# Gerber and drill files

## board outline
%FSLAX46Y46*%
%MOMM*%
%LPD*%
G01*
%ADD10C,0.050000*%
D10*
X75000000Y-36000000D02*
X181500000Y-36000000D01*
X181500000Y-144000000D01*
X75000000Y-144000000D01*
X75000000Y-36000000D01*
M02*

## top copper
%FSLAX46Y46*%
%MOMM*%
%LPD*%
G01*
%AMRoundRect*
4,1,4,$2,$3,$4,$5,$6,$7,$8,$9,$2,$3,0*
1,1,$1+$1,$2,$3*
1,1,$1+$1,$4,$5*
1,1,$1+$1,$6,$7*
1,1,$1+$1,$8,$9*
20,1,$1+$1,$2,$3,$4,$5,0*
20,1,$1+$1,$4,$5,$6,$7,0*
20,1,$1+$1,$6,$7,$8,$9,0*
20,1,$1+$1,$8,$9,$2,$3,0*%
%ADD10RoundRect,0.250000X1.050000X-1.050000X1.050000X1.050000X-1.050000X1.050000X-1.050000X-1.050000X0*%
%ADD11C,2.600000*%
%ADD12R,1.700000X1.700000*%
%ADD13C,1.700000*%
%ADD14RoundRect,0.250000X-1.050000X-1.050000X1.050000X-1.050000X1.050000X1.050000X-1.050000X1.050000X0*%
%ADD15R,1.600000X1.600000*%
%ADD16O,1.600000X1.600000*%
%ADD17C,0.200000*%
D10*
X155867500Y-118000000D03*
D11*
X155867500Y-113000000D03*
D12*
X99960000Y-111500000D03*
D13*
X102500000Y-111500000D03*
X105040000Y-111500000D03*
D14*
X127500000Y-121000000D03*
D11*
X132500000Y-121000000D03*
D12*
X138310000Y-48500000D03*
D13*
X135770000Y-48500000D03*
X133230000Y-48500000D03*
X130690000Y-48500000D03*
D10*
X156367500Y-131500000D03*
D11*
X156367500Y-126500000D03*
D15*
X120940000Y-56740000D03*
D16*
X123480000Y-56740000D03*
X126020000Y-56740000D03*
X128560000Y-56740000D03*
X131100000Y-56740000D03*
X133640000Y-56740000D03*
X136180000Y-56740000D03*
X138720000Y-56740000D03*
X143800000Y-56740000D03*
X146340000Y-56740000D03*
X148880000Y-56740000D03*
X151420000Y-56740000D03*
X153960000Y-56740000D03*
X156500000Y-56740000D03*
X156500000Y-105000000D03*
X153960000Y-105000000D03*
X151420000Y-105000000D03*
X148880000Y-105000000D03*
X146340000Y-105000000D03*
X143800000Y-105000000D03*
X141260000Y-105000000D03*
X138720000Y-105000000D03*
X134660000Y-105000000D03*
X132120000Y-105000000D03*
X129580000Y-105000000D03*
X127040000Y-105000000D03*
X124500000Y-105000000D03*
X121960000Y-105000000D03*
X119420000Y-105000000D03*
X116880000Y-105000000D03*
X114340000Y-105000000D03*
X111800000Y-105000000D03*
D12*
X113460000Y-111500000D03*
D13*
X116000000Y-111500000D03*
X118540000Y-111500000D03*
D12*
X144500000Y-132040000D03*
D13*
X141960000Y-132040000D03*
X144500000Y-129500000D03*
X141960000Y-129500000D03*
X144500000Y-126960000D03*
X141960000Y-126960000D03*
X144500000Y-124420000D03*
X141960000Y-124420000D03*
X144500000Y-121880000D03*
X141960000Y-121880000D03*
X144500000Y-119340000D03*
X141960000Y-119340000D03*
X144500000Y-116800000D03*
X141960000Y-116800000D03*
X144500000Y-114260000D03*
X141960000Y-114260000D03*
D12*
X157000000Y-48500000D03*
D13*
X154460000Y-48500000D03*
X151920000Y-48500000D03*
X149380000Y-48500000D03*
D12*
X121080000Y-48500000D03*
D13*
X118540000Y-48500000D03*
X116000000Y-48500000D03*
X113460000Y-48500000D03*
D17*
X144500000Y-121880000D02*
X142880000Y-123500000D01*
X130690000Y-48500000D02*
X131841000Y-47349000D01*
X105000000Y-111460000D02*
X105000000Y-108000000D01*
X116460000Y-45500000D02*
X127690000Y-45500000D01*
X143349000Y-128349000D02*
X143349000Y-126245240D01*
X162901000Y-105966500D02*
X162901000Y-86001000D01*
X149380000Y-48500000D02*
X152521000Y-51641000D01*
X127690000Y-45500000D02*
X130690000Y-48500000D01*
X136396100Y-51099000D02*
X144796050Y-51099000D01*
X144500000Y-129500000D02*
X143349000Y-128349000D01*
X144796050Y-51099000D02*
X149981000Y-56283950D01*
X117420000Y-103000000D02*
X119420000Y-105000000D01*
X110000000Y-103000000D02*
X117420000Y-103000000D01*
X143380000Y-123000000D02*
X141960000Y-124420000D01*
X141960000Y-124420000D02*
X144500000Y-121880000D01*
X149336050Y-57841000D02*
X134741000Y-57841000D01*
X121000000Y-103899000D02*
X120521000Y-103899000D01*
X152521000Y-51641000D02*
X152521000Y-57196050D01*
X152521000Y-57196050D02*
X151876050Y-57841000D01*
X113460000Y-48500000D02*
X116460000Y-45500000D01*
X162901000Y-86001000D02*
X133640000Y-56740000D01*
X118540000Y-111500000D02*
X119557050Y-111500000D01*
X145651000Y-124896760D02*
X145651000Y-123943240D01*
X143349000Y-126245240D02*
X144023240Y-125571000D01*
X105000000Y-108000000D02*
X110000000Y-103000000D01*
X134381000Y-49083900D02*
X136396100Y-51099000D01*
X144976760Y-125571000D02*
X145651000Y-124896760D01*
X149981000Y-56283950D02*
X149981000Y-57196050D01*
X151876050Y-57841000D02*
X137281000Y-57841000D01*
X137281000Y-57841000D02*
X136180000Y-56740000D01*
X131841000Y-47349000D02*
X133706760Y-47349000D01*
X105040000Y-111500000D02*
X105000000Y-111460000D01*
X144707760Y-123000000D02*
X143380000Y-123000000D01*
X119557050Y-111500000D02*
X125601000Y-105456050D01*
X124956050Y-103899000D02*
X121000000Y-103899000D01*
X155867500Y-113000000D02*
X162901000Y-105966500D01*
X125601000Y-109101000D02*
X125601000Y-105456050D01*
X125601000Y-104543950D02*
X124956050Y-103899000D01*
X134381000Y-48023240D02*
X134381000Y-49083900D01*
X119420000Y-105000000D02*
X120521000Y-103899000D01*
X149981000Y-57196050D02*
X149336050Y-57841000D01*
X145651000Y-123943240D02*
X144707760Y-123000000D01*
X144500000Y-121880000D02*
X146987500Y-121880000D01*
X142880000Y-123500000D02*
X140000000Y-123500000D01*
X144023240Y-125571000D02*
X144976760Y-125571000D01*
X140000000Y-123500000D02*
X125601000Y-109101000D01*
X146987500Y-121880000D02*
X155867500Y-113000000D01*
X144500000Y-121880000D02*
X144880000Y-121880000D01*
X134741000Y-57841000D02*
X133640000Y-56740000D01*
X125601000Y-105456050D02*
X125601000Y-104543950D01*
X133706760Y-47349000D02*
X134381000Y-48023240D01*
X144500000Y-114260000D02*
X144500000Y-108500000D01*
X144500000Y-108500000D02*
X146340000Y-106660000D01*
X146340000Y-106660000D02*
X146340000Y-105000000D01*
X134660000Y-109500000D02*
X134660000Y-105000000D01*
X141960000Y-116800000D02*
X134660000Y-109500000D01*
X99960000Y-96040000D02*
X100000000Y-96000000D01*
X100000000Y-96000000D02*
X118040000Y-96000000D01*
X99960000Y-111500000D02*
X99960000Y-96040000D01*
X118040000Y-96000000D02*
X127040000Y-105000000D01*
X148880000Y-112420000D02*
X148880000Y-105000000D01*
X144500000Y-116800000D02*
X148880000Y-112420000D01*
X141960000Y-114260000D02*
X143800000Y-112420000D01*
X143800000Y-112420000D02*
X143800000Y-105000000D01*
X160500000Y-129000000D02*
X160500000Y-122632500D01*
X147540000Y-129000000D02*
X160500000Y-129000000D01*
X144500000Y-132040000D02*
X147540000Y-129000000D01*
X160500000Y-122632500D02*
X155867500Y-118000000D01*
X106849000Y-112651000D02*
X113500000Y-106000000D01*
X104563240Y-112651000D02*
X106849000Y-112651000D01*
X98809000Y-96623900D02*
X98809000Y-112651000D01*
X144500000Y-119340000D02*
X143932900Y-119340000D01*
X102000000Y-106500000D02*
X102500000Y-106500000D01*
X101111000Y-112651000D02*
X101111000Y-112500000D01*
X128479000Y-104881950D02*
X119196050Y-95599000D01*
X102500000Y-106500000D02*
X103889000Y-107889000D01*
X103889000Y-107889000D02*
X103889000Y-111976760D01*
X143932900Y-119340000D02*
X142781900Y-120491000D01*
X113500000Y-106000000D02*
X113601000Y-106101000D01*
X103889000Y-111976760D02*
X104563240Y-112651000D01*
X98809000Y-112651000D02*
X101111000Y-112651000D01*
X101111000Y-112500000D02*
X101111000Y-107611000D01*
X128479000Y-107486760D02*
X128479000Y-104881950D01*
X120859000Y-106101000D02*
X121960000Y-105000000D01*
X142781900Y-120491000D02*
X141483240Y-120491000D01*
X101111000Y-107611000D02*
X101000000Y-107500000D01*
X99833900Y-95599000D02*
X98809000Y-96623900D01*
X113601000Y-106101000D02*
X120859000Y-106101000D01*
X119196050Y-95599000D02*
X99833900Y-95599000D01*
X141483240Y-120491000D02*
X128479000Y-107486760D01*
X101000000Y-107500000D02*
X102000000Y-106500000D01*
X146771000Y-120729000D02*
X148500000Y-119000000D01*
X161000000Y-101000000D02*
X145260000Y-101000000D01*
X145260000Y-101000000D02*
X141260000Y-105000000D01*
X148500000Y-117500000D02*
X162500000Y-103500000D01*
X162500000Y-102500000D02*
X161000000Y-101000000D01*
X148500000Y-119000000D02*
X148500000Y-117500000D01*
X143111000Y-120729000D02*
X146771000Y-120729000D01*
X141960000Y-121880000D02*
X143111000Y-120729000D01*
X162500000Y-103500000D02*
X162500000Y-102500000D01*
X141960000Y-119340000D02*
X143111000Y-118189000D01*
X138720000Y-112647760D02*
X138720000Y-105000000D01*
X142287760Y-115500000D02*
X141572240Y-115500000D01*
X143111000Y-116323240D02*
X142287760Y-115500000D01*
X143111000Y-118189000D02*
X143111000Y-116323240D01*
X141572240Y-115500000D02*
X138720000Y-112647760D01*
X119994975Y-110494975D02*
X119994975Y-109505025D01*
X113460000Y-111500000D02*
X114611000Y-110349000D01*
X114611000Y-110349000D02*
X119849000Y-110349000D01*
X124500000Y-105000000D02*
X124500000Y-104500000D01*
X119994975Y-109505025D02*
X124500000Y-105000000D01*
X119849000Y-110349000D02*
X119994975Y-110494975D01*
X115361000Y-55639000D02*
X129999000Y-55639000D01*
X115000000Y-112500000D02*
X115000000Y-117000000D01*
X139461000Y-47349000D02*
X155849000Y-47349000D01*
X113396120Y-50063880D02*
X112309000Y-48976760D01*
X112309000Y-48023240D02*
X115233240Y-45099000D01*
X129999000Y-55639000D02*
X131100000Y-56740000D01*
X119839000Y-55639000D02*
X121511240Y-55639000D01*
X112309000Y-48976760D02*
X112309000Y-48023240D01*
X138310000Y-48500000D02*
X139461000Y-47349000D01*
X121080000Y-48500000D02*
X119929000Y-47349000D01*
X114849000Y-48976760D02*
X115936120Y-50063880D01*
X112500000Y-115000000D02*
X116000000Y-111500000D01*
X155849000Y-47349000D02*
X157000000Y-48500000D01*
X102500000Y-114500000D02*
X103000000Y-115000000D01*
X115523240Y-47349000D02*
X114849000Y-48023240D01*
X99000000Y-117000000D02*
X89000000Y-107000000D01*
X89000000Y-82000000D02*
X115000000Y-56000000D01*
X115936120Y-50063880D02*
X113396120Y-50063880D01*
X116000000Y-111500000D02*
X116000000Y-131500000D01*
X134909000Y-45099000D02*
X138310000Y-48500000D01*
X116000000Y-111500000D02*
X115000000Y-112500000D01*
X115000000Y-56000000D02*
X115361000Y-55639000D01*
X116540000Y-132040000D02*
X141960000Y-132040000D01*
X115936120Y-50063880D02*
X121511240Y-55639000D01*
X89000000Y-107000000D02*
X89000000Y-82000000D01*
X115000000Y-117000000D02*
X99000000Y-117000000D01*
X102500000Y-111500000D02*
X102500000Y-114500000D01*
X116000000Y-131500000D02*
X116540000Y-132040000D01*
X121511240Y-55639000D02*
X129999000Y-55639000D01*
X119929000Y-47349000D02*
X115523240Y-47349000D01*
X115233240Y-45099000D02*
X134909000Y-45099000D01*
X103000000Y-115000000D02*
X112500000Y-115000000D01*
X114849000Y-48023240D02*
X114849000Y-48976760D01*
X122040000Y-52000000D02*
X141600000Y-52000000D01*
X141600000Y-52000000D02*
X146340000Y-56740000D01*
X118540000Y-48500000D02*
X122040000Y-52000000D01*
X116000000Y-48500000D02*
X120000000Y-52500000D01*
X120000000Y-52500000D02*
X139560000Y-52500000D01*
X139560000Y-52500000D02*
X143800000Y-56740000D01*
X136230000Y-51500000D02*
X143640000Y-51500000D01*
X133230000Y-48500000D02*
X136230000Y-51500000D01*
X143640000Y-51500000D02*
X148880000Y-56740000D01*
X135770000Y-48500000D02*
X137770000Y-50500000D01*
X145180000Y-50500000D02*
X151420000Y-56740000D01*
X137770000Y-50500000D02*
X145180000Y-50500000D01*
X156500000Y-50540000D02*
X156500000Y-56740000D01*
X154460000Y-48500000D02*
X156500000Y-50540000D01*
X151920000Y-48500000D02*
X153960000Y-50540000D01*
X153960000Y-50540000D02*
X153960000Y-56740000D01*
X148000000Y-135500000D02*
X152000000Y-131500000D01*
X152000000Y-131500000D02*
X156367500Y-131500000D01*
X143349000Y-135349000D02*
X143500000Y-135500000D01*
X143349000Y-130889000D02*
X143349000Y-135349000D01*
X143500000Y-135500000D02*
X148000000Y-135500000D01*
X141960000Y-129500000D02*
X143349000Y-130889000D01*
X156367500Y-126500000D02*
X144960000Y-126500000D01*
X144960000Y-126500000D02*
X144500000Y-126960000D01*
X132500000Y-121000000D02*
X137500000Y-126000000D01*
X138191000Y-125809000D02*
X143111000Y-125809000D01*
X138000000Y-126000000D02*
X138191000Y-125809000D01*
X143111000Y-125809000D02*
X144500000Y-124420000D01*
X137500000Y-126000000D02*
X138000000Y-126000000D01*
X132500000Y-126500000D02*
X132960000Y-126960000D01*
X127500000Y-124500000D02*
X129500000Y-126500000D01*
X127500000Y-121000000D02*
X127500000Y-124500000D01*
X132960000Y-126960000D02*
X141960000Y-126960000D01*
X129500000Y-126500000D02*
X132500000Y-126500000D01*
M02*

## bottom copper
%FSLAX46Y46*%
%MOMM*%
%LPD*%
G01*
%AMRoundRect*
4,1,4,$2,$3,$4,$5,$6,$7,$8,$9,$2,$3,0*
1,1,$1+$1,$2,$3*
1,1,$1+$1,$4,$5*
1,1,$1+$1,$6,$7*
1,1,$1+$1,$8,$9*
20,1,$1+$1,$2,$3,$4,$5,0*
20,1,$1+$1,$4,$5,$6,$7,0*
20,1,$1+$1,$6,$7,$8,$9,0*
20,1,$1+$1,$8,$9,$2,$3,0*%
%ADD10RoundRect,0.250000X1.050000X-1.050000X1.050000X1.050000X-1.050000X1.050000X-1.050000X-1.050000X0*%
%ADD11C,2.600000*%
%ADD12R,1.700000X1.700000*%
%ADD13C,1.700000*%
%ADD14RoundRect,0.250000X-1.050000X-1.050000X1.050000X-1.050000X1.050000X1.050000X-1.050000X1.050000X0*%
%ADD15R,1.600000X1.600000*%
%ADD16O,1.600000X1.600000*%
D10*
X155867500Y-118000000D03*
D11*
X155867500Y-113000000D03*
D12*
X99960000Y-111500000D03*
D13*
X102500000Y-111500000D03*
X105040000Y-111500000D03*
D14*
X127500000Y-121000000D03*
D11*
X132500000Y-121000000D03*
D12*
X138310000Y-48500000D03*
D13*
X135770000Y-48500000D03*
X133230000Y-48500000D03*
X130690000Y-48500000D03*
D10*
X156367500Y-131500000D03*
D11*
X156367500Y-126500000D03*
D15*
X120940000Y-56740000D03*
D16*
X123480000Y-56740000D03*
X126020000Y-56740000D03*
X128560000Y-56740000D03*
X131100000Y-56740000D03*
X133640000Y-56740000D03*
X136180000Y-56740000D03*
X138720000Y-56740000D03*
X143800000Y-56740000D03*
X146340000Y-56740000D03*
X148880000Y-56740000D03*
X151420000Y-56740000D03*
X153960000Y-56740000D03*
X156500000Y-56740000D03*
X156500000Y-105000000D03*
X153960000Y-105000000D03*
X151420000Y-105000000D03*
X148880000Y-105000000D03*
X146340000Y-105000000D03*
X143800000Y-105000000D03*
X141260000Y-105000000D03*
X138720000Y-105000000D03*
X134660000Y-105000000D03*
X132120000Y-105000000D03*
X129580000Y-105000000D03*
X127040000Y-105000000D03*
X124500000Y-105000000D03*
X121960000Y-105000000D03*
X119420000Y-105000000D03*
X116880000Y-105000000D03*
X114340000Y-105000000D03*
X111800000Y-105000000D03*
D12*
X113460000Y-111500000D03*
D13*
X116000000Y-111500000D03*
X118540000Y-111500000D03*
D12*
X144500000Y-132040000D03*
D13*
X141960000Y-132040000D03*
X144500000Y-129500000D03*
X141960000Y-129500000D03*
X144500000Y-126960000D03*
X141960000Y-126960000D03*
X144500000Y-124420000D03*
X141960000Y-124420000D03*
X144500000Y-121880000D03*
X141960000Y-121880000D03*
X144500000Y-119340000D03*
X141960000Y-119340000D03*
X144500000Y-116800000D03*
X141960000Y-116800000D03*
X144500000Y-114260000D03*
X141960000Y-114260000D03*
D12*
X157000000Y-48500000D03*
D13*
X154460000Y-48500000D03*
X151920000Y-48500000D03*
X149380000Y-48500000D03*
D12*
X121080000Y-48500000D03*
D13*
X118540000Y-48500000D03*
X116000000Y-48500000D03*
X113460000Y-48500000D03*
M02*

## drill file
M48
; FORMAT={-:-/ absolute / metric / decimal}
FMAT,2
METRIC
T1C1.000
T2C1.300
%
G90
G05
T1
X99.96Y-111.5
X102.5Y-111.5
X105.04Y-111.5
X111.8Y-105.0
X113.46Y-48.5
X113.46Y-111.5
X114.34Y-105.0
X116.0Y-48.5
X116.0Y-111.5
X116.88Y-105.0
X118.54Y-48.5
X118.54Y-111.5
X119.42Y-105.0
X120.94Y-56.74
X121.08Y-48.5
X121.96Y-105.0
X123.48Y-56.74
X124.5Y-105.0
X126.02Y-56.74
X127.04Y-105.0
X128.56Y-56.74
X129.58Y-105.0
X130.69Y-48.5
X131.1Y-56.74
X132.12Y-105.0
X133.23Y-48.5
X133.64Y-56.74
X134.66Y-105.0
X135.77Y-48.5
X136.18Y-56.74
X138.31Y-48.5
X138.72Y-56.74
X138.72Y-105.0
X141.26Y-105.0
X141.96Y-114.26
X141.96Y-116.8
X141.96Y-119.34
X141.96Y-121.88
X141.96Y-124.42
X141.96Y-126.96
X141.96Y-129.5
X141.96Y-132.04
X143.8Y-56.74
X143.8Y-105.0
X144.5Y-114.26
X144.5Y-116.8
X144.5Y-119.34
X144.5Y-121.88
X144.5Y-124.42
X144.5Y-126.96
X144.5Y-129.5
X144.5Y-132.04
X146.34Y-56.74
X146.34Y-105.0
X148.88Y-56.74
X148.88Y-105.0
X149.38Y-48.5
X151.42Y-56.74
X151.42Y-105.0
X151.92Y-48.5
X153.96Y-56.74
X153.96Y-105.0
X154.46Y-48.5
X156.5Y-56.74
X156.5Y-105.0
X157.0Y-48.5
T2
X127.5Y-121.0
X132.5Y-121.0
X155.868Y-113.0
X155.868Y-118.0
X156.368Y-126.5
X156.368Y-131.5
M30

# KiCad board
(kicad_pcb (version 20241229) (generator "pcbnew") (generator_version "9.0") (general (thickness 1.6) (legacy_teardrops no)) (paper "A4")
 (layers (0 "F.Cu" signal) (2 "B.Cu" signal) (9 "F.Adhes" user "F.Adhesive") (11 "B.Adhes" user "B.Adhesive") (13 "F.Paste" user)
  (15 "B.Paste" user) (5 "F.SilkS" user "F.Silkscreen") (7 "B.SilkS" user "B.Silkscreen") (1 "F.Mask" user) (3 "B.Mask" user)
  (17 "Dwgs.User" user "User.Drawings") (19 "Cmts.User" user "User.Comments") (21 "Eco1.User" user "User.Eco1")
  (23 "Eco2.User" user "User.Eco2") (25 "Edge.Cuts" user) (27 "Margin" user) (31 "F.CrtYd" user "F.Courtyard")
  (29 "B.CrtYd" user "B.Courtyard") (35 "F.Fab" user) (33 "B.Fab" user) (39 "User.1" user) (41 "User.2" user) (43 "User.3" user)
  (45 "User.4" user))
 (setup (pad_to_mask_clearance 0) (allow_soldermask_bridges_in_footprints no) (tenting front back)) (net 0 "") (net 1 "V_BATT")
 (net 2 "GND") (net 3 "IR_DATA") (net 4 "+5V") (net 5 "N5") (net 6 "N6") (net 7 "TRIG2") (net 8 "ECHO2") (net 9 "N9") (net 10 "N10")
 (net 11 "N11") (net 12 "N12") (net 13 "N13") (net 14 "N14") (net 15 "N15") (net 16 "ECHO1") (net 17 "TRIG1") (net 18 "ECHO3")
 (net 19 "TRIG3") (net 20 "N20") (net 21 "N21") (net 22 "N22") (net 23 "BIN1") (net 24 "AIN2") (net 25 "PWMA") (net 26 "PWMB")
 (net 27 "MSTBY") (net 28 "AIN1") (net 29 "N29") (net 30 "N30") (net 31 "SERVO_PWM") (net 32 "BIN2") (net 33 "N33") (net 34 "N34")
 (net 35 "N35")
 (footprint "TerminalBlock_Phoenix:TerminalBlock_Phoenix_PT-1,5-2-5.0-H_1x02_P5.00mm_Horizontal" (layer "F.Cu") (at 155.8675 118 90)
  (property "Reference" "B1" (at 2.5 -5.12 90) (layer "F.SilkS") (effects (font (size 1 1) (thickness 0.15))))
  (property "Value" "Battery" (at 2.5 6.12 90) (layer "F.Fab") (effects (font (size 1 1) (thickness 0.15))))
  (pad "1" thru_hole roundrect (at 0 0 90) (size 2.6 2.6) (drill 1.3) (layers "*.Cu" "*.Mask") (remove_unused_layers no)
   (roundrect_rratio 0.096154) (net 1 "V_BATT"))
  (pad "2" thru_hole circle (at 5 0 90) (size 2.6 2.6) (drill 1.3) (layers "*.Cu" "*.Mask") (remove_unused_layers no) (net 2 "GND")))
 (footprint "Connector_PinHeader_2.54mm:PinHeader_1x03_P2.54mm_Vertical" (layer "F.Cu") (at 99.96 111.5 90)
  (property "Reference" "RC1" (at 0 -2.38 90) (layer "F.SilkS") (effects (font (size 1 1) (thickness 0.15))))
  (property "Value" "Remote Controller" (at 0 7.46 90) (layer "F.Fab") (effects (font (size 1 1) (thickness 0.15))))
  (pad "1" thru_hole rect (at 0 0 90) (size 1.7 1.7) (drill 1) (layers "*.Cu" "*.Mask") (remove_unused_layers no) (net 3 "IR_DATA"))
  (pad "2" thru_hole circle (at 0 2.54 90) (size 1.7 1.7) (drill 1) (layers "*.Cu" "*.Mask") (remove_unused_layers no) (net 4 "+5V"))
  (pad "3" thru_hole circle (at 0 5.08 90) (size 1.7 1.7) (drill 1) (layers "*.Cu" "*.Mask") (remove_unused_layers no) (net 2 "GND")))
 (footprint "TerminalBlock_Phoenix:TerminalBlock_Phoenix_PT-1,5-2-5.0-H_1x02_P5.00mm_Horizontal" (layer "F.Cu") (at 127.5 121)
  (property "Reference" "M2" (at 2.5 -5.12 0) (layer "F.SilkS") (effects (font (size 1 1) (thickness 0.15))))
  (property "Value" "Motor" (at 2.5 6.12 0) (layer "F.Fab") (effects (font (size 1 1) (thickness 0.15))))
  (pad "1" thru_hole roundrect (at 0 0) (size 2.6 2.6) (drill 1.3) (layers "*.Cu" "*.Mask") (remove_unused_layers no)
   (roundrect_rratio 0.096154) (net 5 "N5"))
  (pad "2" thru_hole circle (at 5 0) (size 2.6 2.6) (drill 1.3) (layers "*.Cu" "*.Mask") (remove_unused_layers no) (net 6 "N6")))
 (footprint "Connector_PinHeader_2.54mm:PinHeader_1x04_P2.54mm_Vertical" (layer "F.Cu") (at 138.31 48.5 -90)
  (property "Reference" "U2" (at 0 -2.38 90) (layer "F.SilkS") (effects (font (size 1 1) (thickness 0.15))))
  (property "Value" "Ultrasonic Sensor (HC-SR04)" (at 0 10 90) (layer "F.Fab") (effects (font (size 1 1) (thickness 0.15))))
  (pad "1" thru_hole rect (at 0 0 270) (size 1.7 1.7) (drill 1) (layers "*.Cu" "*.Mask") (remove_unused_layers no) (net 4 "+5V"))
  (pad "2" thru_hole circle (at 0 2.54 270) (size 1.7 1.7) (drill 1) (layers "*.Cu" "*.Mask") (remove_unused_layers no) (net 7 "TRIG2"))
  (pad "3" thru_hole circle (at 0 5.08 270) (size 1.7 1.7) (drill 1) (layers "*.Cu" "*.Mask") (remove_unused_layers no) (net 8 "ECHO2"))
  (pad "4" thru_hole circle (at 0 7.62 270) (size 1.7 1.7) (drill 1) (layers "*.Cu" "*.Mask") (remove_unused_layers no) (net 2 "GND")))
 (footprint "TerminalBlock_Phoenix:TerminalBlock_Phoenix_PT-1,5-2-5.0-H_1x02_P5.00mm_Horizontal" (layer "F.Cu") (at 156.3675 131.5 90)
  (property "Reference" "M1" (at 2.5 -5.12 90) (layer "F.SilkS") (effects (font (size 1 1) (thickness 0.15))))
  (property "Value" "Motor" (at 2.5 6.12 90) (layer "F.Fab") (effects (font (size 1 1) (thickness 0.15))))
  (pad "1" thru_hole roundrect (at 0 0 90) (size 2.6 2.6) (drill 1.3) (layers "*.Cu" "*.Mask") (remove_unused_layers no)
   (roundrect_rratio 0.096154) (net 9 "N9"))
  (pad "2" thru_hole circle (at 5 0 90) (size 2.6 2.6) (drill 1.3) (layers "*.Cu" "*.Mask") (remove_unused_layers no) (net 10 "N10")))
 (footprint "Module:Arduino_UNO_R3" (layer "F.Cu") (at 120.94 56.74)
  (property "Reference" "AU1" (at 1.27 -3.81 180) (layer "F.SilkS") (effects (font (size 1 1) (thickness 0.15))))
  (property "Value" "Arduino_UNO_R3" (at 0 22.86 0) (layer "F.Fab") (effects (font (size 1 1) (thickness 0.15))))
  (pad "1" thru_hole rect (at 0 0 90) (size 1.6 1.6) (drill 1) (layers "*.Cu" "*.Mask") (remove_unused_layers no) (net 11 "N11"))
  (pad "2" thru_hole oval (at 2.54 0 90) (size 1.6 1.6) (drill 1) (layers "*.Cu" "*.Mask") (remove_unused_layers no) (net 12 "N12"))
  (pad "3" thru_hole oval (at 5.08 0 90) (size 1.6 1.6) (drill 1) (layers "*.Cu" "*.Mask") (remove_unused_layers no) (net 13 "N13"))
  (pad "4" thru_hole oval (at 7.62 0 90) (size 1.6 1.6) (drill 1) (layers "*.Cu" "*.Mask") (remove_unused_layers no) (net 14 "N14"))
  (pad "5" thru_hole oval (at 10.16 0 90) (size 1.6 1.6) (drill 1) (layers "*.Cu" "*.Mask") (remove_unused_layers no) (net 4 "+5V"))
  (pad "6" thru_hole oval (at 12.7 0 90) (size 1.6 1.6) (drill 1) (layers "*.Cu" "*.Mask") (remove_unused_layers no) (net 2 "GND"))
  (pad "7" thru_hole oval (at 15.24 0 90) (size 1.6 1.6) (drill 1) (layers "*.Cu" "*.Mask") (remove_unused_layers no) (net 2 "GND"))
  (pad "8" thru_hole oval (at 17.78 0 90) (size 1.6 1.6) (drill 1) (layers "*.Cu" "*.Mask") (remove_unused_layers no) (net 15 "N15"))
  (pad "9" thru_hole oval (at 22.86 0 90) (size 1.6 1.6) (drill 1) (layers "*.Cu" "*.Mask") (remove_unused_layers no) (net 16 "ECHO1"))
  (pad "10" thru_hole oval (at 25.4 0 90) (size 1.6 1.6) (drill 1) (layers "*.Cu" "*.Mask") (remove_unused_layers no) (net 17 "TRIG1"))
  (pad "11" thru_hole oval (at 27.94 0 90) (size 1.6 1.6) (drill 1) (layers "*.Cu" "*.Mask") (remove_unused_layers no) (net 8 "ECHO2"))
  (pad "12" thru_hole oval (at 30.48 0 90) (size 1.6 1.6) (drill 1) (layers "*.Cu" "*.Mask") (remove_unused_layers no) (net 7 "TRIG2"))
  (pad "13" thru_hole oval (at 33.02 0 90) (size 1.6 1.6) (drill 1) (layers "*.Cu" "*.Mask") (remove_unused_layers no) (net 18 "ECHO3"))
  (pad "14" thru_hole oval (at 35.56 0 90) (size 1.6 1.6) (drill 1) (layers "*.Cu" "*.Mask") (remove_unused_layers no) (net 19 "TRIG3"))
  (pad "15" thru_hole oval (at 35.56 48.26 90) (size 1.6 1.6) (drill 1) (layers "*.Cu" "*.Mask") (remove_unused_layers no) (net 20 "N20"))
  (pad "16" thru_hole oval (at 33.02 48.26 90) (size 1.6 1.6) (drill 1) (layers "*.Cu" "*.Mask") (remove_unused_layers no) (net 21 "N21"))
  (pad "17" thru_hole oval (at 30.48 48.26 90) (size 1.6 1.6) (drill 1) (layers "*.Cu" "*.Mask") (remove_unused_layers no) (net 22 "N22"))
  (pad "18" thru_hole oval (at 27.94 48.26 90) (size 1.6 1.6) (drill 1) (layers "*.Cu" "*.Mask") (remove_unused_layers no) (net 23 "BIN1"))
  (pad "19" thru_hole oval (at 25.4 48.26 90) (size 1.6 1.6) (drill 1) (layers "*.Cu" "*.Mask") (remove_unused_layers no) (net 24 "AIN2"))
  (pad "20" thru_hole oval (at 22.86 48.26 90) (size 1.6 1.6) (drill 1) (layers "*.Cu" "*.Mask") (remove_unused_layers no) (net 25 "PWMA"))
  (pad "21" thru_hole oval (at 20.32 48.26 90) (size 1.6 1.6) (drill 1) (layers "*.Cu" "*.Mask") (remove_unused_layers no) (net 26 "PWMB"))
  (pad "22" thru_hole oval (at 17.78 48.26 90) (size 1.6 1.6) (drill 1) (layers "*.Cu" "*.Mask") (remove_unused_layers no) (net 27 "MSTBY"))
  (pad "23" thru_hole oval (at 13.72 48.26 90) (size 1.6 1.6) (drill 1) (layers "*.Cu" "*.Mask") (remove_unused_layers no) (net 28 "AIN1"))
  (pad "24" thru_hole oval (at 11.18 48.26 90) (size 1.6 1.6) (drill 1) (layers "*.Cu" "*.Mask") (remove_unused_layers no) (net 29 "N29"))
  (pad "25" thru_hole oval (at 8.64 48.26 90) (size 1.6 1.6) (drill 1) (layers "*.Cu" "*.Mask") (remove_unused_layers no) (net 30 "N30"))
  (pad "26" thru_hole oval (at 6.1 48.26 90) (size 1.6 1.6) (drill 1) (layers "*.Cu" "*.Mask") (remove_unused_layers no) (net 3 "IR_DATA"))
  (pad "27" thru_hole oval (at 3.56 48.26 90) (size 1.6 1.6) (drill 1) (layers "*.Cu" "*.Mask") (remove_unused_layers no)
   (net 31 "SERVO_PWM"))
  (pad "28" thru_hole oval (at 1.02 48.26 90) (size 1.6 1.6) (drill 1) (layers "*.Cu" "*.Mask") (remove_unused_layers no) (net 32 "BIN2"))
  (pad "29" thru_hole oval (at -1.52 48.26 90) (size 1.6 1.6) (drill 1) (layers "*.Cu" "*.Mask") (remove_unused_layers no) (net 2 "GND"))
  (pad "30" thru_hole oval (at -4.06 48.26 90) (size 1.6 1.6) (drill 1) (layers "*.Cu" "*.Mask") (remove_unused_layers no) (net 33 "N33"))
  (pad "31" thru_hole oval (at -6.6 48.26 90) (size 1.6 1.6) (drill 1) (layers "*.Cu" "*.Mask") (remove_unused_layers no) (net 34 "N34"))
  (pad "32" thru_hole oval (at -9.14 48.26 90) (size 1.6 1.6) (drill 1) (layers "*.Cu" "*.Mask") (remove_unused_layers no) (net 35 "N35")))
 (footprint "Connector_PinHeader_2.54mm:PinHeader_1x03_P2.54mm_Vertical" (layer "F.Cu") (at 113.46 111.5 90)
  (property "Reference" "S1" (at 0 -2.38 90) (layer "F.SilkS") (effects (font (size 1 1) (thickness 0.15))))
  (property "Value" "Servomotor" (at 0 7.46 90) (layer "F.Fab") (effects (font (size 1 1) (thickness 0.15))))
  (pad "1" thru_hole rect (at 0 0 90) (size 1.7 1.7) (drill 1) (layers "*.Cu" "*.Mask") (remove_unused_layers no) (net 31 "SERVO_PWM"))
  (pad "2" thru_hole circle (at 0 2.54 90) (size 1.7 1.7) (drill 1) (layers "*.Cu" "*.Mask") (remove_unused_layers no) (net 4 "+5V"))
  (pad "3" thru_hole circle (at 0 5.08 90) (size 1.7 1.7) (drill 1) (layers "*.Cu" "*.Mask") (remove_unused_layers no) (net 2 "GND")))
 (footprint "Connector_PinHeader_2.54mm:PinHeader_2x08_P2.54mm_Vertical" (layer "F.Cu") (at 144.5 132.04 180)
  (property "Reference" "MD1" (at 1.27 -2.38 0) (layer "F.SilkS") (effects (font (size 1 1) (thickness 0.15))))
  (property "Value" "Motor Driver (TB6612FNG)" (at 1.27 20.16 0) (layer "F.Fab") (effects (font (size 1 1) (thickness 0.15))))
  (pad "1" thru_hole rect (at 0 0 180) (size 1.7 1.7) (drill 1) (layers "*.Cu" "*.Mask") (remove_unused_layers no) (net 1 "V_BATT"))
  (pad "2" thru_hole circle (at 2.54 0 180) (size 1.7 1.7) (drill 1) (layers "*.Cu" "*.Mask") (remove_unused_layers no) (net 4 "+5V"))
  (pad "3" thru_hole circle (at 0 2.54 180) (size 1.7 1.7) (drill 1) (layers "*.Cu" "*.Mask") (remove_unused_layers no) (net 2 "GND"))
  (pad "4" thru_hole circle (at 2.54 2.54 180) (size 1.7 1.7) (drill 1) (layers "*.Cu" "*.Mask") (remove_unused_layers no) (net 9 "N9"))
  (pad "5" thru_hole circle (at 0 5.08 180) (size 1.7 1.7) (drill 1) (layers "*.Cu" "*.Mask") (remove_unused_layers no) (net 10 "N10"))
  (pad "6" thru_hole circle (at 2.54 5.08 180) (size 1.7 1.7) (drill 1) (layers "*.Cu" "*.Mask") (remove_unused_layers no) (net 5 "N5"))
  (pad "7" thru_hole circle (at 0 7.62 180) (size 1.7 1.7) (drill 1) (layers "*.Cu" "*.Mask") (remove_unused_layers no) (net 6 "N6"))
  (pad "8" thru_hole circle (at 2.54 7.62 180) (size 1.7 1.7) (drill 1) (layers "*.Cu" "*.Mask") (remove_unused_layers no) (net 2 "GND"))
  (pad "9" thru_hole circle (at 0 10.16 180) (size 1.7 1.7) (drill 1) (layers "*.Cu" "*.Mask") (remove_unused_layers no) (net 2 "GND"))
  (pad "10" thru_hole circle (at 2.54 10.16 180) (size 1.7 1.7) (drill 1) (layers "*.Cu" "*.Mask") (remove_unused_layers no) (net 26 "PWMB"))
  (pad "11" thru_hole circle (at 0 12.7 180) (size 1.7 1.7) (drill 1) (layers "*.Cu" "*.Mask") (remove_unused_layers no) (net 32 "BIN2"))
  (pad "12" thru_hole circle (at 2.54 12.7 180) (size 1.7 1.7) (drill 1) (layers "*.Cu" "*.Mask") (remove_unused_layers no) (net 27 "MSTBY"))
  (pad "13" thru_hole circle (at 0 15.24 180) (size 1.7 1.7) (drill 1) (layers "*.Cu" "*.Mask") (remove_unused_layers no) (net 23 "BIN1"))
  (pad "14" thru_hole circle (at 2.54 15.24 180) (size 1.7 1.7) (drill 1) (layers "*.Cu" "*.Mask") (remove_unused_layers no) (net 28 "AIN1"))
  (pad "15" thru_hole circle (at 0 17.78 180) (size 1.7 1.7) (drill 1) (layers "*.Cu" "*.Mask") (remove_unused_layers no) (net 24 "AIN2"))
  (pad "16" thru_hole circle (at 2.54 17.78 180) (size 1.7 1.7) (drill 1) (layers "*.Cu" "*.Mask") (remove_unused_layers no) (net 25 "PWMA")))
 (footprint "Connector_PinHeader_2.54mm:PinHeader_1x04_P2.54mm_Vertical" (layer "F.Cu") (at 157 48.5 -90)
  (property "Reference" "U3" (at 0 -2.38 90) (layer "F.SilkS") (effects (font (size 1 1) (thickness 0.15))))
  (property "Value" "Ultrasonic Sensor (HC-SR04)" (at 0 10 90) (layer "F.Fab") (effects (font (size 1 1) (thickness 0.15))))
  (pad "1" thru_hole rect (at 0 0 270) (size 1.7 1.7) (drill 1) (layers "*.Cu" "*.Mask") (remove_unused_layers no) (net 4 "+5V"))
  (pad "2" thru_hole circle (at 0 2.54 270) (size 1.7 1.7) (drill 1) (layers "*.Cu" "*.Mask") (remove_unused_layers no) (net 19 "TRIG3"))
  (pad "3" thru_hole circle (at 0 5.08 270) (size 1.7 1.7) (drill 1) (layers "*.Cu" "*.Mask") (remove_unused_layers no) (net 18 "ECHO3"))
  (pad "4" thru_hole circle (at 0 7.62 270) (size 1.7 1.7) (drill 1) (layers "*.Cu" "*.Mask") (remove_unused_layers no) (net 2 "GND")))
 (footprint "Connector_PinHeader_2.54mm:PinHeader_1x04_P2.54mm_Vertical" (layer "F.Cu") (at 121.08 48.5 -90)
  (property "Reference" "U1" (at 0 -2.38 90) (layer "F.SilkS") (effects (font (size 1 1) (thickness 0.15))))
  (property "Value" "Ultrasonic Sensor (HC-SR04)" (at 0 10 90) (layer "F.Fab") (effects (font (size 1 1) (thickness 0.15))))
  (pad "1" thru_hole rect (at 0 0 270) (size 1.7 1.7) (drill 1) (layers "*.Cu" "*.Mask") (remove_unused_layers no) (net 4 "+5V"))
  (pad "2" thru_hole circle (at 0 2.54 270) (size 1.7 1.7) (drill 1) (layers "*.Cu" "*.Mask") (remove_unused_layers no) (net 17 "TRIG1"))
  (pad "3" thru_hole circle (at 0 5.08 270) (size 1.7 1.7) (drill 1) (layers "*.Cu" "*.Mask") (remove_unused_layers no) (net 16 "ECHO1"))
  (pad "4" thru_hole circle (at 0 7.62 270) (size 1.7 1.7) (drill 1) (layers "*.Cu" "*.Mask") (remove_unused_layers no) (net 2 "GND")))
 (gr_rect (start 75 36) (end 181.5 144) (stroke (width 0.05) (type default)) (fill no) (layer "Edge.Cuts"))
 (segment (start 144.5 121.88) (end 142.88 123.5) (width 0.2) (layer "F.Cu") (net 2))
 (segment (start 130.69 48.5) (end 131.841 47.349) (width 0.2) (layer "F.Cu") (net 2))
 (segment (start 105 111.46) (end 105 108) (width 0.2) (layer "F.Cu") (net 2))
 (segment (start 116.46 45.5) (end 127.69 45.5) (width 0.2) (layer "F.Cu") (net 2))
 (segment (start 143.349 128.349) (end 143.349 126.24524) (width 0.2) (layer "F.Cu") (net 2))
 (segment (start 162.901 105.9665) (end 162.901 86.001) (width 0.2) (layer "F.Cu") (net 2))
 (segment (start 149.38 48.5) (end 152.521 51.641) (width 0.2) (layer "F.Cu") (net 2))
 (segment (start 127.69 45.5) (end 130.69 48.5) (width 0.2) (layer "F.Cu") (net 2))
 (segment (start 136.3961 51.099) (end 144.79605 51.099) (width 0.2) (layer "F.Cu") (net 2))
 (segment (start 144.5 129.5) (end 143.349 128.349) (width 0.2) (layer "F.Cu") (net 2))
 (segment (start 144.79605 51.099) (end 149.981 56.28395) (width 0.2) (layer "F.Cu") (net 2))
 (segment (start 117.42 103) (end 119.42 105) (width 0.2) (layer "F.Cu") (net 2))
 (segment (start 110 103) (end 117.42 103) (width 0.2) (layer "F.Cu") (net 2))
 (segment (start 143.38 123) (end 141.96 124.42) (width 0.2) (layer "F.Cu") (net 2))
 (segment (start 141.96 124.42) (end 144.5 121.88) (width 0.2) (layer "F.Cu") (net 2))
 (segment (start 149.33605 57.841) (end 134.741 57.841) (width 0.2) (layer "F.Cu") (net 2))
 (segment (start 121 103.899) (end 120.521 103.899) (width 0.2) (layer "F.Cu") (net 2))
 (segment (start 152.521 51.641) (end 152.521 57.19605) (width 0.2) (layer "F.Cu") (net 2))
 (segment (start 152.521 57.19605) (end 151.87605 57.841) (width 0.2) (layer "F.Cu") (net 2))
 (segment (start 113.46 48.5) (end 116.46 45.5) (width 0.2) (layer "F.Cu") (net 2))
 (segment (start 162.901 86.001) (end 133.64 56.74) (width 0.2) (layer "F.Cu") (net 2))
 (segment (start 118.54 111.5) (end 119.55705 111.5) (width 0.2) (layer "F.Cu") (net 2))
 (segment (start 145.651 124.89676) (end 145.651 123.94324) (width 0.2) (layer "F.Cu") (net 2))
 (segment (start 143.349 126.24524) (end 144.02324 125.571) (width 0.2) (layer "F.Cu") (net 2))
 (segment (start 105 108) (end 110 103) (width 0.2) (layer "F.Cu") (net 2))
 (segment (start 134.381 49.0839) (end 136.3961 51.099) (width 0.2) (layer "F.Cu") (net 2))
 (segment (start 144.97676 125.571) (end 145.651 124.89676) (width 0.2) (layer "F.Cu") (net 2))
 (segment (start 149.981 56.28395) (end 149.981 57.19605) (width 0.2) (layer "F.Cu") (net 2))
 (segment (start 151.87605 57.841) (end 137.281 57.841) (width 0.2) (layer "F.Cu") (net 2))
 (segment (start 137.281 57.841) (end 136.18 56.74) (width 0.2) (layer "F.Cu") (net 2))
 (segment (start 131.841 47.349) (end 133.70676 47.349) (width 0.2) (layer "F.Cu") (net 2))
 (segment (start 105.04 111.5) (end 105 111.46) (width 0.2) (layer "F.Cu") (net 2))
 (segment (start 144.70776 123) (end 143.38 123) (width 0.2) (layer "F.Cu") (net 2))
 (segment (start 119.55705 111.5) (end 125.601 105.45605) (width 0.2) (layer "F.Cu") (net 2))
 (segment (start 124.95605 103.899) (end 121 103.899) (width 0.2) (layer "F.Cu") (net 2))
 (segment (start 155.8675 113) (end 162.901 105.9665) (width 0.2) (layer "F.Cu") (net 2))
 (segment (start 125.601 109.101) (end 125.601 105.45605) (width 0.2) (layer "F.Cu") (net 2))
 (segment (start 125.601 104.54395) (end 124.95605 103.899) (width 0.2) (layer "F.Cu") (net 2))
 (segment (start 134.381 48.02324) (end 134.381 49.0839) (width 0.2) (layer "F.Cu") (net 2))
 (segment (start 119.42 105) (end 120.521 103.899) (width 0.2) (layer "F.Cu") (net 2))
 (segment (start 149.981 57.19605) (end 149.33605 57.841) (width 0.2) (layer "F.Cu") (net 2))
 (segment (start 145.651 123.94324) (end 144.70776 123) (width 0.2) (layer "F.Cu") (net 2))
 (segment (start 144.5 121.88) (end 146.9875 121.88) (width 0.2) (layer "F.Cu") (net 2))
 (segment (start 142.88 123.5) (end 140 123.5) (width 0.2) (layer "F.Cu") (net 2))
 (segment (start 144.02324 125.571) (end 144.97676 125.571) (width 0.2) (layer "F.Cu") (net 2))
 (segment (start 140 123.5) (end 125.601 109.101) (width 0.2) (layer "F.Cu") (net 2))
 (segment (start 146.9875 121.88) (end 155.8675 113) (width 0.2) (layer "F.Cu") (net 2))
 (segment (start 144.5 121.88) (end 144.88 121.88) (width 0.2) (layer "F.Cu") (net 2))
 (segment (start 134.741 57.841) (end 133.64 56.74) (width 0.2) (layer "F.Cu") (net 2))
 (segment (start 125.601 105.45605) (end 125.601 104.54395) (width 0.2) (layer "F.Cu") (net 2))
 (segment (start 133.70676 47.349) (end 134.381 48.02324) (width 0.2) (layer "F.Cu") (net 2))
 (segment (start 144.5 114.26) (end 144.5 108.5) (width 0.2) (layer "F.Cu") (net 24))
 (segment (start 144.5 108.5) (end 146.34 106.66) (width 0.2) (layer "F.Cu") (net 24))
 (segment (start 146.34 106.66) (end 146.34 105) (width 0.2) (layer "F.Cu") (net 24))
 (segment (start 134.66 109.5) (end 134.66 105) (width 0.2) (layer "F.Cu") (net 28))
 (segment (start 141.96 116.8) (end 134.66 109.5) (width 0.2) (layer "F.Cu") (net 28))
 (segment (start 99.96 96.04) (end 100 96) (width 0.2) (layer "F.Cu") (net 3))
 (segment (start 100 96) (end 118.04 96) (width 0.2) (layer "F.Cu") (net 3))
 (segment (start 99.96 111.5) (end 99.96 96.04) (width 0.2) (layer "F.Cu") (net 3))
 (segment (start 118.04 96) (end 127.04 105) (width 0.2) (layer "F.Cu") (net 3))
 (segment (start 148.88 112.42) (end 148.88 105) (width 0.2) (layer "F.Cu") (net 23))
 (segment (start 144.5 116.8) (end 148.88 112.42) (width 0.2) (layer "F.Cu") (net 23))
 (segment (start 141.96 114.26) (end 143.8 112.42) (width 0.2) (layer "F.Cu") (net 25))
 (segment (start 143.8 112.42) (end 143.8 105) (width 0.2) (layer "F.Cu") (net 25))
 (segment (start 160.5 129) (end 160.5 122.6325) (width 0.2) (layer "F.Cu") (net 1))
 (segment (start 147.54 129) (end 160.5 129) (width 0.2) (layer "F.Cu") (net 1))
 (segment (start 144.5 132.04) (end 147.54 129) (width 0.2) (layer "F.Cu") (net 1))
 (segment (start 160.5 122.6325) (end 155.8675 118) (width 0.2) (layer "F.Cu") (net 1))
 (segment (start 106.849 112.651) (end 113.5 106) (width 0.2) (layer "F.Cu") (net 32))
 (segment (start 104.56324 112.651) (end 106.849 112.651) (width 0.2) (layer "F.Cu") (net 32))
 (segment (start 98.809 96.6239) (end 98.809 112.651) (width 0.2) (layer "F.Cu") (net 32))
 (segment (start 144.5 119.34) (end 143.9329 119.34) (width 0.2) (layer "F.Cu") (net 32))
 (segment (start 102 106.5) (end 102.5 106.5) (width 0.2) (layer "F.Cu") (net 32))
 (segment (start 101.111 112.651) (end 101.111 112.5) (width 0.2) (layer "F.Cu") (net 32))
 (segment (start 128.479 104.88195) (end 119.19605 95.599) (width 0.2) (layer "F.Cu") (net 32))
 (segment (start 102.5 106.5) (end 103.889 107.889) (width 0.2) (layer "F.Cu") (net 32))
 (segment (start 103.889 107.889) (end 103.889 111.97676) (width 0.2) (layer "F.Cu") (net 32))
 (segment (start 143.9329 119.34) (end 142.7819 120.491) (width 0.2) (layer "F.Cu") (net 32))
 (segment (start 113.5 106) (end 113.601 106.101) (width 0.2) (layer "F.Cu") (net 32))
 (segment (start 103.889 111.97676) (end 104.56324 112.651) (width 0.2) (layer "F.Cu") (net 32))
 (segment (start 98.809 112.651) (end 101.111 112.651) (width 0.2) (layer "F.Cu") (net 32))
 (segment (start 101.111 112.5) (end 101.111 107.611) (width 0.2) (layer "F.Cu") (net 32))
 (segment (start 128.479 107.48676) (end 128.479 104.88195) (width 0.2) (layer "F.Cu") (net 32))
 (segment (start 120.859 106.101) (end 121.96 105) (width 0.2) (layer "F.Cu") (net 32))
 (segment (start 142.7819 120.491) (end 141.48324 120.491) (width 0.2) (layer "F.Cu") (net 32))
 (segment (start 101.111 107.611) (end 101 107.5) (width 0.2) (layer "F.Cu") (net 32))
 (segment (start 99.8339 95.599) (end 98.809 96.6239) (width 0.2) (layer "F.Cu") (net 32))
 (segment (start 113.601 106.101) (end 120.859 106.101) (width 0.2) (layer "F.Cu") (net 32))
 (segment (start 119.19605 95.599) (end 99.8339 95.599) (width 0.2) (layer "F.Cu") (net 32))
 (segment (start 141.48324 120.491) (end 128.479 107.48676) (width 0.2) (layer "F.Cu") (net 32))
 (segment (start 101 107.5) (end 102 106.5) (width 0.2) (layer "F.Cu") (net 32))
 (segment (start 146.771 120.729) (end 148.5 119) (width 0.2) (layer "F.Cu") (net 26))
 (segment (start 161 101) (end 145.26 101) (width 0.2) (layer "F.Cu") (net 26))
 (segment (start 145.26 101) (end 141.26 105) (width 0.2) (layer "F.Cu") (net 26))
 (segment (start 148.5 117.5) (end 162.5 103.5) (width 0.2) (layer "F.Cu") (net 26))
 (segment (start 162.5 102.5) (end 161 101) (width 0.2) (layer "F.Cu") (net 26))
 (segment (start 148.5 119) (end 148.5 117.5) (width 0.2) (layer "F.Cu") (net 26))
 (segment (start 143.111 120.729) (end 146.771 120.729) (width 0.2) (layer "F.Cu") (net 26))
 (segment (start 141.96 121.88) (end 143.111 120.729) (width 0.2) (layer "F.Cu") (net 26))
 (segment (start 162.5 103.5) (end 162.5 102.5) (width 0.2) (layer "F.Cu") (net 26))
 (segment (start 141.96 119.34) (end 143.111 118.189) (width 0.2) (layer "F.Cu") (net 27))
 (segment (start 138.72 112.64776) (end 138.72 105) (width 0.2) (layer "F.Cu") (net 27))
 (segment (start 142.28776 115.5) (end 141.57224 115.5) (width 0.2) (layer "F.Cu") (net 27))
 (segment (start 143.111 116.32324) (end 142.28776 115.5) (width 0.2) (layer "F.Cu") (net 27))
 (segment (start 143.111 118.189) (end 143.111 116.32324) (width 0.2) (layer "F.Cu") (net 27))
 (segment (start 141.57224 115.5) (end 138.72 112.64776) (width 0.2) (layer "F.Cu") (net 27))
 (segment (start 119.994975 110.494975) (end 119.994975 109.505025) (width 0.2) (layer "F.Cu") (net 31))
 (segment (start 113.46 111.5) (end 114.611 110.349) (width 0.2) (layer "F.Cu") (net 31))
 (segment (start 114.611 110.349) (end 119.849 110.349) (width 0.2) (layer "F.Cu") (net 31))
 (segment (start 124.5 105) (end 124.5 104.5) (width 0.2) (layer "F.Cu") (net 31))
 (segment (start 119.994975 109.505025) (end 124.5 105) (width 0.2) (layer "F.Cu") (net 31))
 (segment (start 119.849 110.349) (end 119.994975 110.494975) (width 0.2) (layer "F.Cu") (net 31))
 (segment (start 115.361 55.639) (end 129.999 55.639) (width 0.2) (layer "F.Cu") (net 4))
 (segment (start 115 112.5) (end 115 117) (width 0.2) (layer "F.Cu") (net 4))
 (segment (start 139.461 47.349) (end 155.849 47.349) (width 0.2) (layer "F.Cu") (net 4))
 (segment (start 113.39612 50.06388) (end 112.309 48.97676) (width 0.2) (layer "F.Cu") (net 4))
 (segment (start 112.309 48.02324) (end 115.23324 45.099) (width 0.2) (layer "F.Cu") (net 4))
 (segment (start 129.999 55.639) (end 131.1 56.74) (width 0.2) (layer "F.Cu") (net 4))
 (segment (start 119.839 55.639) (end 121.51124 55.639) (width 0.2) (layer "F.Cu") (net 4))
 (segment (start 112.309 48.97676) (end 112.309 48.02324) (width 0.2) (layer "F.Cu") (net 4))
 (segment (start 138.31 48.5) (end 139.461 47.349) (width 0.2) (layer "F.Cu") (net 4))
 (segment (start 121.08 48.5) (end 119.929 47.349) (width 0.2) (layer "F.Cu") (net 4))
 (segment (start 114.849 48.97676) (end 115.93612 50.06388) (width 0.2) (layer "F.Cu") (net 4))
 (segment (start 112.5 115) (end 116 111.5) (width 0.2) (layer "F.Cu") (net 4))
 (segment (start 155.849 47.349) (end 157 48.5) (width 0.2) (layer "F.Cu") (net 4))
 (segment (start 102.5 114.5) (end 103 115) (width 0.2) (layer "F.Cu") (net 4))
 (segment (start 115.52324 47.349) (end 114.849 48.02324) (width 0.2) (layer "F.Cu") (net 4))
 (segment (start 99 117) (end 89 107) (width 0.2) (layer "F.Cu") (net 4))
 (segment (start 89 82) (end 115 56) (width 0.2) (layer "F.Cu") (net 4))
 (segment (start 115.93612 50.06388) (end 113.39612 50.06388) (width 0.2) (layer "F.Cu") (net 4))
 (segment (start 116 111.5) (end 116 131.5) (width 0.2) (layer "F.Cu") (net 4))
 (segment (start 134.909 45.099) (end 138.31 48.5) (width 0.2) (layer "F.Cu") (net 4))
 (segment (start 116 111.5) (end 115 112.5) (width 0.2) (layer "F.Cu") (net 4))
 (segment (start 115 56) (end 115.361 55.639) (width 0.2) (layer "F.Cu") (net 4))
 (segment (start 116.54 132.04) (end 141.96 132.04) (width 0.2) (layer "F.Cu") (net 4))
 (segment (start 115.93612 50.06388) (end 121.51124 55.639) (width 0.2) (layer "F.Cu") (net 4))
 (segment (start 89 107) (end 89 82) (width 0.2) (layer "F.Cu") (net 4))
 (segment (start 115 117) (end 99 117) (width 0.2) (layer "F.Cu") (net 4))
 (segment (start 102.5 111.5) (end 102.5 114.5) (width 0.2) (layer "F.Cu") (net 4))
 (segment (start 116 131.5) (end 116.54 132.04) (width 0.2) (layer "F.Cu") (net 4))
 (segment (start 121.51124 55.639) (end 129.999 55.639) (width 0.2) (layer "F.Cu") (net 4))
 (segment (start 119.929 47.349) (end 115.52324 47.349) (width 0.2) (layer "F.Cu") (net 4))
 (segment (start 115.23324 45.099) (end 134.909 45.099) (width 0.2) (layer "F.Cu") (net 4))
 (segment (start 103 115) (end 112.5 115) (width 0.2) (layer "F.Cu") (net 4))
 (segment (start 114.849 48.02324) (end 114.849 48.97676) (width 0.2) (layer "F.Cu") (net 4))
 (segment (start 122.04 52) (end 141.6 52) (width 0.2) (layer "F.Cu") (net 17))
 (segment (start 141.6 52) (end 146.34 56.74) (width 0.2) (layer "F.Cu") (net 17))
 (segment (start 118.54 48.5) (end 122.04 52) (width 0.2) (layer "F.Cu") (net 17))
 (segment (start 116 48.5) (end 120 52.5) (width 0.2) (layer "F.Cu") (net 16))
 (segment (start 120 52.5) (end 139.56 52.5) (width 0.2) (layer "F.Cu") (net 16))
 (segment (start 139.56 52.5) (end 143.8 56.74) (width 0.2) (layer "F.Cu") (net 16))
 (segment (start 136.23 51.5) (end 143.64 51.5) (width 0.2) (layer "F.Cu") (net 8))
 (segment (start 133.23 48.5) (end 136.23 51.5) (width 0.2) (layer "F.Cu") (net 8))
 (segment (start 143.64 51.5) (end 148.88 56.74) (width 0.2) (layer "F.Cu") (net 8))
 (segment (start 135.77 48.5) (end 137.77 50.5) (width 0.2) (layer "F.Cu") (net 7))
 (segment (start 145.18 50.5) (end 151.42 56.74) (width 0.2) (layer "F.Cu") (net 7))
 (segment (start 137.77 50.5) (end 145.18 50.5) (width 0.2) (layer "F.Cu") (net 7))
 (segment (start 156.5 50.54) (end 156.5 56.74) (width 0.2) (layer "F.Cu") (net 19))
 (segment (start 154.46 48.5) (end 156.5 50.54) (width 0.2) (layer "F.Cu") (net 19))
 (segment (start 151.92 48.5) (end 153.96 50.54) (width 0.2) (layer "F.Cu") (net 18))
 (segment (start 153.96 50.54) (end 153.96 56.74) (width 0.2) (layer "F.Cu") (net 18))
 (segment (start 148 135.5) (end 152 131.5) (width 0.2) (layer "F.Cu") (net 9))
 (segment (start 152 131.5) (end 156.3675 131.5) (width 0.2) (layer "F.Cu") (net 9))
 (segment (start 143.349 135.349) (end 143.5 135.5) (width 0.2) (layer "F.Cu") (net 9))
 (segment (start 143.349 130.889) (end 143.349 135.349) (width 0.2) (layer "F.Cu") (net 9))
 (segment (start 143.5 135.5) (end 148 135.5) (width 0.2) (layer "F.Cu") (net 9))
 (segment (start 141.96 129.5) (end 143.349 130.889) (width 0.2) (layer "F.Cu") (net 9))
 (segment (start 156.3675 126.5) (end 144.96 126.5) (width 0.2) (layer "F.Cu") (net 10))
 (segment (start 144.96 126.5) (end 144.5 126.96) (width 0.2) (layer "F.Cu") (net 10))
 (segment (start 132.5 121) (end 137.5 126) (width 0.2) (layer "F.Cu") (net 6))
 (segment (start 138.191 125.809) (end 143.111 125.809) (width 0.2) (layer "F.Cu") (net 6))
 (segment (start 138 126) (end 138.191 125.809) (width 0.2) (layer "F.Cu") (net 6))
 (segment (start 143.111 125.809) (end 144.5 124.42) (width 0.2) (layer "F.Cu") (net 6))
 (segment (start 137.5 126) (end 138 126) (width 0.2) (layer "F.Cu") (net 6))
 (segment (start 132.5 126.5) (end 132.96 126.96) (width 0.2) (layer "F.Cu") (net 5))
 (segment (start 127.5 124.5) (end 129.5 126.5) (width 0.2) (layer "F.Cu") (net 5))
 (segment (start 127.5 121) (end 127.5 124.5) (width 0.2) (layer "F.Cu") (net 5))
 (segment (start 132.96 126.96) (end 141.96 126.96) (width 0.2) (layer "F.Cu") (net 5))
 (segment (start 129.5 126.5) (end 132.5 126.5) (width 0.2) (layer "F.Cu") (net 5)))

